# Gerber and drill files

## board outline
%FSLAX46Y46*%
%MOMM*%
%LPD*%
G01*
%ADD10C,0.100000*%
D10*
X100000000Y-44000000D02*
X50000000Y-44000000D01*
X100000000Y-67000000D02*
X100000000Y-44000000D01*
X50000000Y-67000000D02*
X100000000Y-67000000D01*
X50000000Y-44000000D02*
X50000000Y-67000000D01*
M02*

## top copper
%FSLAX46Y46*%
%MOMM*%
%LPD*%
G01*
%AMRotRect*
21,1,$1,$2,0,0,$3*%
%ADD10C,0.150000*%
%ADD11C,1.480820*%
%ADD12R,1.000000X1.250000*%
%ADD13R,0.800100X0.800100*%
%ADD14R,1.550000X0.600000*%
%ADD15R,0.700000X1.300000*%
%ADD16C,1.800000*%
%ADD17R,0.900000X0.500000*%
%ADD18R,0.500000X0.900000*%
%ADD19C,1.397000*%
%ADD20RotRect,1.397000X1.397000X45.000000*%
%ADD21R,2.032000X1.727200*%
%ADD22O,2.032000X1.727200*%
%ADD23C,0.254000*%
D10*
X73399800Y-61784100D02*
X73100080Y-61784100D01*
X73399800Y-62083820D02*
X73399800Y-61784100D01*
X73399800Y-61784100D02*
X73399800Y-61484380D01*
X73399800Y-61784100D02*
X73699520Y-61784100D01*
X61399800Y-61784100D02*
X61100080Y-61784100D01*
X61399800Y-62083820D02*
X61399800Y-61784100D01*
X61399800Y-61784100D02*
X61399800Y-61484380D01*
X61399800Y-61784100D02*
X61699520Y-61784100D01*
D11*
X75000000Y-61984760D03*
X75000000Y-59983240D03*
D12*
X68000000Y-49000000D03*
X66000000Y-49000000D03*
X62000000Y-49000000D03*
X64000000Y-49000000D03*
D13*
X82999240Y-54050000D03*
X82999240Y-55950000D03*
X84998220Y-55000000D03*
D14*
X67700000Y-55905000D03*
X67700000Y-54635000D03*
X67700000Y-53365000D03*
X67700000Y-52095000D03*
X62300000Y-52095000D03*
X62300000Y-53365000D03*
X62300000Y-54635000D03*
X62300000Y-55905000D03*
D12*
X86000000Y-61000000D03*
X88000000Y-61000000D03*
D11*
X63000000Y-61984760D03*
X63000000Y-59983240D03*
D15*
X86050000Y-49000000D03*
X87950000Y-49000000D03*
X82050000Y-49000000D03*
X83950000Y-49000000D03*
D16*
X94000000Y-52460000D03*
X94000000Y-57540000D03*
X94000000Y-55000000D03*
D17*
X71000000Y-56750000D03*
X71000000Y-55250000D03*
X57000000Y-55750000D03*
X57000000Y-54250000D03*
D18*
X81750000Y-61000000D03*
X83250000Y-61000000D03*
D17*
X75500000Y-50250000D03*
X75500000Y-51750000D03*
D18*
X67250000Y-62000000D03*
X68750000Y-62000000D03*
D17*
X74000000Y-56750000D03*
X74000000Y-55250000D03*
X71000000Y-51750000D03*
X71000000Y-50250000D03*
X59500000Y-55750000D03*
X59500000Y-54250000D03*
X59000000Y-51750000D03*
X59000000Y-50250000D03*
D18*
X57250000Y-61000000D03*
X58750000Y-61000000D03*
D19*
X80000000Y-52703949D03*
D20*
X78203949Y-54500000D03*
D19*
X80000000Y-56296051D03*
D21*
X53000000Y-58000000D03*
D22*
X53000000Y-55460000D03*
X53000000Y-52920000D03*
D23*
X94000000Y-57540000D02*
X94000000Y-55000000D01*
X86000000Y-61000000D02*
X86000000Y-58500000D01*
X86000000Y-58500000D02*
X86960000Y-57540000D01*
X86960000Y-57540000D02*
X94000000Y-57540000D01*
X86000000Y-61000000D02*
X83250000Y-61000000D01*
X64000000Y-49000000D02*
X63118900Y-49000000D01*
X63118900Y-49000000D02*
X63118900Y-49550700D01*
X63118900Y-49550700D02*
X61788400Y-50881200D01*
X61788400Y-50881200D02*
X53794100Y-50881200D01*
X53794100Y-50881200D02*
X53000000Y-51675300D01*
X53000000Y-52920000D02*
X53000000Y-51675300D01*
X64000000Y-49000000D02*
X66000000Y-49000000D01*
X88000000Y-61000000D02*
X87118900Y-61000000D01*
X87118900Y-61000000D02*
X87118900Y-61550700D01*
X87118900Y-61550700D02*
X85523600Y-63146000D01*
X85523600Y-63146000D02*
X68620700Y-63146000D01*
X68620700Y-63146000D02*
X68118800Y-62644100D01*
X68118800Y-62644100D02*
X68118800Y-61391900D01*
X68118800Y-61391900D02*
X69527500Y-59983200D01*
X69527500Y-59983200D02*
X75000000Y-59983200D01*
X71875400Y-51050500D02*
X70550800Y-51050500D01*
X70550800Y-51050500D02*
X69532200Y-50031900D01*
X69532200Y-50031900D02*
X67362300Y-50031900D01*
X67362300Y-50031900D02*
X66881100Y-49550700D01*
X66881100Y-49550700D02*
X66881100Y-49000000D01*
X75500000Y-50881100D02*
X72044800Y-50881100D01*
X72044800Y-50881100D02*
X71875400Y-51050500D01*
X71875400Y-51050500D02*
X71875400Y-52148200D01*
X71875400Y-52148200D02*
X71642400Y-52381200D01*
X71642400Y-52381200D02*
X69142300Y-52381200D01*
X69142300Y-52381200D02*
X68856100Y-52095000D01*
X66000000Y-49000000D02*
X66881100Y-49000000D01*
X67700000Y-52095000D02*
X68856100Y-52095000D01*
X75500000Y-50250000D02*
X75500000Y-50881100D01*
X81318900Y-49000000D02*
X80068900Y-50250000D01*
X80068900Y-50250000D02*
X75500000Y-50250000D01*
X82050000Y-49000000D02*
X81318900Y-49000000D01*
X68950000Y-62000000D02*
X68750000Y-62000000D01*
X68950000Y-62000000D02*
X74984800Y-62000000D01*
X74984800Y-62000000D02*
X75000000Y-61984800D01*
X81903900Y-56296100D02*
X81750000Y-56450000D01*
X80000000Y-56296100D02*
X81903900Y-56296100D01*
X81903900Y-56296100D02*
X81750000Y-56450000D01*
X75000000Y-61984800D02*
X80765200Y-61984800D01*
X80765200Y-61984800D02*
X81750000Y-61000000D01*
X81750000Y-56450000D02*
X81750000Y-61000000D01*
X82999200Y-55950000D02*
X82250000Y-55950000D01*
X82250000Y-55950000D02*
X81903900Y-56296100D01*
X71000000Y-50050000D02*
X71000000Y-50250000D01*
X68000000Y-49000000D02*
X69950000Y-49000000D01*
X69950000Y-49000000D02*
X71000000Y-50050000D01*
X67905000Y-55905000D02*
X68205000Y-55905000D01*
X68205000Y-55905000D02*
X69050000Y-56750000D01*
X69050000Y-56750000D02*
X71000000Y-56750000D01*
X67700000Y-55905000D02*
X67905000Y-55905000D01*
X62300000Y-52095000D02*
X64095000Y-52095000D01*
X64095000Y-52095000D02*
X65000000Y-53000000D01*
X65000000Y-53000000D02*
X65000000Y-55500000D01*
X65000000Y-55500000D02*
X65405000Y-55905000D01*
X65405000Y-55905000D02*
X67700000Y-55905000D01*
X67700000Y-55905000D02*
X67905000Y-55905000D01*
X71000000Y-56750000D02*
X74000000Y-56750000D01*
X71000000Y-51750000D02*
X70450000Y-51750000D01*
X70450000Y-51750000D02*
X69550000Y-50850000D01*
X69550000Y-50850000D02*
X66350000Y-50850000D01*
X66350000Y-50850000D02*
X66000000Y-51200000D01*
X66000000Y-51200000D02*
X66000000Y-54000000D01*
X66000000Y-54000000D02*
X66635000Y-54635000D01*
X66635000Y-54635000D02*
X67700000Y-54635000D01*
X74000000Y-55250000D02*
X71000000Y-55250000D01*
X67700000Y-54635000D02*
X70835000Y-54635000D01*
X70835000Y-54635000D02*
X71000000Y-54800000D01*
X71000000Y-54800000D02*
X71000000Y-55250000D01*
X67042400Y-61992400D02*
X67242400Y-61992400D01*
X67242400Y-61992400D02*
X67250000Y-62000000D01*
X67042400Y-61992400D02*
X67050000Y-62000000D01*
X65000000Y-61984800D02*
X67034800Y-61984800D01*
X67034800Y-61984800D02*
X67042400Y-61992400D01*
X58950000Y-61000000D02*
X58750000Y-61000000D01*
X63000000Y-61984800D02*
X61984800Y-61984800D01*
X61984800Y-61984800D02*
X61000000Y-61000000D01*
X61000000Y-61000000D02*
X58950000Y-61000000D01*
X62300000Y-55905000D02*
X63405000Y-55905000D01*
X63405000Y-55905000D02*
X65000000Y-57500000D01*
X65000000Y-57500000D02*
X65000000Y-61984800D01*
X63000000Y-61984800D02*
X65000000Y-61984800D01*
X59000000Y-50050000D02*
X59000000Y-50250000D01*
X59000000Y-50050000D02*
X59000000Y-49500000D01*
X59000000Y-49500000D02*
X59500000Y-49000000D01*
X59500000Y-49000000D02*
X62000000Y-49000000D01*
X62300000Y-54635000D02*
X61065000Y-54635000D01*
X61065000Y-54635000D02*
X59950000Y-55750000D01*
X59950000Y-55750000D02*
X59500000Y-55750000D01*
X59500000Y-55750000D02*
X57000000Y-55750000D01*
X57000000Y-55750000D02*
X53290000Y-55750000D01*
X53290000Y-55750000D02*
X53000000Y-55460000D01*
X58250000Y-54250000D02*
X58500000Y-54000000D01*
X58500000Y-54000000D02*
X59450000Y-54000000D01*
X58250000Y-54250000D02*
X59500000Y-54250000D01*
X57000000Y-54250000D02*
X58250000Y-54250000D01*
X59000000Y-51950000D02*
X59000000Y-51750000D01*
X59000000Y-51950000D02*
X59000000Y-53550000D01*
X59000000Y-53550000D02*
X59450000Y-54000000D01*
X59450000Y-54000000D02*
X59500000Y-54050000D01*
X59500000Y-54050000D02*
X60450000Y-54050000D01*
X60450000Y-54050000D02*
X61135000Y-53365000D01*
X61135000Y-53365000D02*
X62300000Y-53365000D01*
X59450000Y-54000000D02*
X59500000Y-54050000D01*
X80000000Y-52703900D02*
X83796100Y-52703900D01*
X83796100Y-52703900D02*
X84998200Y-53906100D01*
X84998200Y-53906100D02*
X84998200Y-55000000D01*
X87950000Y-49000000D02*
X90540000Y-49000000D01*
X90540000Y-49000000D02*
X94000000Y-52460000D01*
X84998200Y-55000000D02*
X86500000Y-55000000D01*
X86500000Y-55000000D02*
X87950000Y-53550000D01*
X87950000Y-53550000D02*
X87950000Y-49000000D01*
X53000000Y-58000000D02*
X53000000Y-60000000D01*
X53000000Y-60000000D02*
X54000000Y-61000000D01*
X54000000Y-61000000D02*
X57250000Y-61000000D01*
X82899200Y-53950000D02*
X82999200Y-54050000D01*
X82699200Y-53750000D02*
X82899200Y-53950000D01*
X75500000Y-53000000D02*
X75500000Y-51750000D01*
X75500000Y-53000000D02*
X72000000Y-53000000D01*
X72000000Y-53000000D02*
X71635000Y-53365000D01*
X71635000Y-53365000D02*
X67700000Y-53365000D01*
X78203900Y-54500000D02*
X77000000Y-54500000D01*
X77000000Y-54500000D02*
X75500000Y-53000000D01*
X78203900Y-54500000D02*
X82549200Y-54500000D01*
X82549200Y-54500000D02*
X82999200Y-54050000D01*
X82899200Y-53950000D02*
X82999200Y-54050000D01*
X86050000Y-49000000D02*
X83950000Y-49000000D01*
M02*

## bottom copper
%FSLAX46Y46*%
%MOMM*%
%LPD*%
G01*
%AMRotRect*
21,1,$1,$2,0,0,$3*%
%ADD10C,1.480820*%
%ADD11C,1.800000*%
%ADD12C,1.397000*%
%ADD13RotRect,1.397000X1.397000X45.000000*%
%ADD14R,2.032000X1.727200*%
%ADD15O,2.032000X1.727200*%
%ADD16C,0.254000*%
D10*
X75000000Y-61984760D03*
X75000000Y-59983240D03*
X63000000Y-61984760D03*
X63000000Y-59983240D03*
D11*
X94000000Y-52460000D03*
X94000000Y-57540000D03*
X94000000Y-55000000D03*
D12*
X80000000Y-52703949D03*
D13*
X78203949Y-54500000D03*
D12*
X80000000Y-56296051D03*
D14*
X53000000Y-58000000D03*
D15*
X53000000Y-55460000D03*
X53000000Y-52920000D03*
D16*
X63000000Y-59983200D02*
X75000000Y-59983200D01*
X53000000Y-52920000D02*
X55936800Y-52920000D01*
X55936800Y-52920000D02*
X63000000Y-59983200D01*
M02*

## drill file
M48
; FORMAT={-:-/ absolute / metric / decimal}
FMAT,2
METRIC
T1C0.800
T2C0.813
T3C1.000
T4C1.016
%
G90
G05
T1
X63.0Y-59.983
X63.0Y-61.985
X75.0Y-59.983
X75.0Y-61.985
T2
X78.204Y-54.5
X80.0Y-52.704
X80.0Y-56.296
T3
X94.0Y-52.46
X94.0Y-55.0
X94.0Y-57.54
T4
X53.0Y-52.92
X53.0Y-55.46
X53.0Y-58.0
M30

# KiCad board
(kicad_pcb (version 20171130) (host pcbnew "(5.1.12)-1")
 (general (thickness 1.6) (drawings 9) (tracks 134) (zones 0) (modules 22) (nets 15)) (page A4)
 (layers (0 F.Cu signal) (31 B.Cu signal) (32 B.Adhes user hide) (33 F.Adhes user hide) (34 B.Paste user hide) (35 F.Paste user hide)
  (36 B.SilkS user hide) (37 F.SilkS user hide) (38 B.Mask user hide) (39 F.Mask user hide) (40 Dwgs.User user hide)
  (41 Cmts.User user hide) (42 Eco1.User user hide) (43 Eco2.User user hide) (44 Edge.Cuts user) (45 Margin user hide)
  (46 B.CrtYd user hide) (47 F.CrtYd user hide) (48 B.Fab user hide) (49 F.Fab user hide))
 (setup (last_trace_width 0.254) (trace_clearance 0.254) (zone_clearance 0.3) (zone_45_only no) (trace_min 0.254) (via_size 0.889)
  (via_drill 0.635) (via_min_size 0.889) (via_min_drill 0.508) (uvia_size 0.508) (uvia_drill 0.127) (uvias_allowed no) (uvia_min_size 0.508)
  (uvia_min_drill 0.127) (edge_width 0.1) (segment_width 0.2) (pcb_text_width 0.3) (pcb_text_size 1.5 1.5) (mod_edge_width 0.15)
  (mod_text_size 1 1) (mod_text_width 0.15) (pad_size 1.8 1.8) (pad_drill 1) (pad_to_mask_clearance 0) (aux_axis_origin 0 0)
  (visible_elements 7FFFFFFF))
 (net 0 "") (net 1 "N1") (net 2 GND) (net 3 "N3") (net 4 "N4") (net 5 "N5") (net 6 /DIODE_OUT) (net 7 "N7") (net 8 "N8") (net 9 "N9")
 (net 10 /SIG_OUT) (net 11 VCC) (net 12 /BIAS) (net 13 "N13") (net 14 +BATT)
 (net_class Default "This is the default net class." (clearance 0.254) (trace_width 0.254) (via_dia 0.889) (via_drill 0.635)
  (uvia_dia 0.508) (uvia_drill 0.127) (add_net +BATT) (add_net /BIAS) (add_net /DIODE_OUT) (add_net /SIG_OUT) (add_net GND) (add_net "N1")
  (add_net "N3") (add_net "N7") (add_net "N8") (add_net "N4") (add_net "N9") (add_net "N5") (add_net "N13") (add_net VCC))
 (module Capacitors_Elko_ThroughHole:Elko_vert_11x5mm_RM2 (layer F.Cu) (at 75 62 90)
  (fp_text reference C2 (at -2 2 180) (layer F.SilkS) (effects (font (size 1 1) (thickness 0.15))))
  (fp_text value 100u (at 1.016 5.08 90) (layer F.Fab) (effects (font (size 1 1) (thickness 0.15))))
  (fp_line (start 0.2159 -1.6002) (end 0.2159 -1.89992) (layer F.Cu) (width 0.15))
  (fp_line (start -0.08382 -1.6002) (end 0.2159 -1.6002) (layer F.Cu) (width 0.15))
  (fp_line (start 0.2159 -1.6002) (end 0.51562 -1.6002) (layer F.Cu) (width 0.15))
  (fp_line (start 0.2159 -1.6002) (end 0.2159 -1.30048) (layer F.Cu) (width 0.15))
  (pad 1 thru_hole circle (at 0.01524 0 90) (size 1.48082 1.48082) (drill 0.8001) (layers *.Cu *.Mask F.SilkS) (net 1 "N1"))
  (pad 2 thru_hole circle (at 2.01676 0 90) (size 1.48082 1.48082) (drill 0.8001) (layers *.Cu *.Mask F.SilkS) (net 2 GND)))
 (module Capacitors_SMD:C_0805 (layer F.Cu) (at 67 49 180)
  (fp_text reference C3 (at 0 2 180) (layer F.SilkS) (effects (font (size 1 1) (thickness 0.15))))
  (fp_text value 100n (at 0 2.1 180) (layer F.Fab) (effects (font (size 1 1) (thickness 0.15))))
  (pad 1 smd rect (at -1 0 180) (size 1 1.25) (layers F.Cu F.Paste F.Mask) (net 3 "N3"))
  (pad 2 smd rect (at 1 0 180) (size 1 1.25) (layers F.Cu F.Paste F.Mask) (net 2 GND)))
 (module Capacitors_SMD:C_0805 (layer F.Cu) (at 63 49)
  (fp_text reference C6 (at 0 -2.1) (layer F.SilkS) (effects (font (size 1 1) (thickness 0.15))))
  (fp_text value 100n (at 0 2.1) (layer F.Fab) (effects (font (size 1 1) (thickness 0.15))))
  (pad 1 smd rect (at -1 0) (size 1 1.25) (layers F.Cu F.Paste F.Mask) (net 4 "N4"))
  (pad 2 smd rect (at 1 0) (size 1 1.25) (layers F.Cu F.Paste F.Mask) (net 2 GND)))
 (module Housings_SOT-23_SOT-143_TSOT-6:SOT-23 (layer F.Cu) (at 84 55 270)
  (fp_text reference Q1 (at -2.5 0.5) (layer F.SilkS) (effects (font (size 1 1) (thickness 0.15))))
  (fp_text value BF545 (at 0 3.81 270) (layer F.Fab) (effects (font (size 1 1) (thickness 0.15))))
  (pad 1 smd rect (at -0.95 1.00076 270) (size 0.8001 0.8001) (layers F.Cu F.Paste F.Mask) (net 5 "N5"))
  (pad 2 smd rect (at 0.95 1.00076 270) (size 0.8001 0.8001) (layers F.Cu F.Paste F.Mask) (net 1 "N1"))
  (pad 3 smd rect (at 0 -0.99822 270) (size 0.8001 0.8001) (layers F.Cu F.Paste F.Mask) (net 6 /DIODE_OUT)))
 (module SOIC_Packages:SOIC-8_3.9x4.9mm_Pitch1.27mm (layer F.Cu) (at 65 54 180)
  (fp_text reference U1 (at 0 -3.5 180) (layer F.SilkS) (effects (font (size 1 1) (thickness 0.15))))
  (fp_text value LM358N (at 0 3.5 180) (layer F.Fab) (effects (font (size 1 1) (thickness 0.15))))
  (pad 1 smd rect (at -2.7 -1.905 180) (size 1.55 0.6) (layers F.Cu F.Paste F.Mask) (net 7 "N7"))
  (pad 2 smd rect (at -2.7 -0.635 180) (size 1.55 0.6) (layers F.Cu F.Paste F.Mask) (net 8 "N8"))
  (pad 3 smd rect (at -2.7 0.635 180) (size 1.55 0.6) (layers F.Cu F.Paste F.Mask) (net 5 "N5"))
  (pad 4 smd rect (at -2.7 1.905 180) (size 1.55 0.6) (layers F.Cu F.Paste F.Mask) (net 2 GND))
  (pad 5 smd rect (at 2.7 1.905 180) (size 1.55 0.6) (layers F.Cu F.Paste F.Mask) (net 7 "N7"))
  (pad 6 smd rect (at 2.7 0.635 180) (size 1.55 0.6) (layers F.Cu F.Paste F.Mask) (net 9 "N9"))
  (pad 7 smd rect (at 2.7 -0.635 180) (size 1.55 0.6) (layers F.Cu F.Paste F.Mask) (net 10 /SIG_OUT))
  (pad 8 smd rect (at 2.7 -1.905 180) (size 1.55 0.6) (layers F.Cu F.Paste F.Mask) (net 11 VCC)))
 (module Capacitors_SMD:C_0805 (layer F.Cu) (at 87 61)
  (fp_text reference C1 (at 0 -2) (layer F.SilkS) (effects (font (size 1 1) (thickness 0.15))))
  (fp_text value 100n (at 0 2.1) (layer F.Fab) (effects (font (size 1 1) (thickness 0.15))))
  (pad 1 smd rect (at -1 0) (size 1 1.25) (layers F.Cu F.Paste F.Mask) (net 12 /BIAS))
  (pad 2 smd rect (at 1 0) (size 1 1.25) (layers F.Cu F.Paste F.Mask) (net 2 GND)))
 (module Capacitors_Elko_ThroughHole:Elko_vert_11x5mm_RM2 (layer F.Cu) (at 63 62 90)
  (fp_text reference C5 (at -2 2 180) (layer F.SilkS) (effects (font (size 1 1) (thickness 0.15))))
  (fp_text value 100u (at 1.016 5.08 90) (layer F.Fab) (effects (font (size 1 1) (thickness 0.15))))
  (fp_line (start 0.2159 -1.6002) (end 0.2159 -1.89992) (layer F.Cu) (width 0.15))
  (fp_line (start -0.08382 -1.6002) (end 0.2159 -1.6002) (layer F.Cu) (width 0.15))
  (fp_line (start 0.2159 -1.6002) (end 0.51562 -1.6002) (layer F.Cu) (width 0.15))
  (fp_line (start 0.2159 -1.6002) (end 0.2159 -1.30048) (layer F.Cu) (width 0.15))
  (pad 1 thru_hole circle (at 0.01524 0 90) (size 1.48082 1.48082) (drill 0.8001) (layers *.Cu *.Mask F.SilkS) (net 11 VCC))
  (pad 2 thru_hole circle (at 2.01676 0 90) (size 1.48082 1.48082) (drill 0.8001) (layers *.Cu *.Mask F.SilkS) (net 2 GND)))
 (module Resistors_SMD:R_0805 (layer F.Cu) (at 87 49)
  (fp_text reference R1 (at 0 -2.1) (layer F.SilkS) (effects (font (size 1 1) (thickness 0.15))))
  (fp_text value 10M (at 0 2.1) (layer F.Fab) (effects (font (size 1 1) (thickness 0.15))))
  (pad 1 smd rect (at -0.95 0) (size 0.7 1.3) (layers F.Cu F.Paste F.Mask) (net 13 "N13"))
  (pad 2 smd rect (at 0.95 0) (size 0.7 1.3) (layers F.Cu F.Paste F.Mask) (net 6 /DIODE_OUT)))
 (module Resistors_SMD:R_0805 (layer F.Cu) (at 83 49)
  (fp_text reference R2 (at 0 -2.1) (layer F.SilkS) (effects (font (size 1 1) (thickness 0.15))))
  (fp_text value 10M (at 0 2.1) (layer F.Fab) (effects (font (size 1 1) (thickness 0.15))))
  (pad 1 smd rect (at -0.95 0) (size 0.7 1.3) (layers F.Cu F.Paste F.Mask) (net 2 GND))
  (pad 2 smd rect (at 0.95 0) (size 0.7 1.3) (layers F.Cu F.Paste F.Mask) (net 13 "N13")))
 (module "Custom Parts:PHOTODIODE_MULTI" (layer F.Cu) (at 94 55)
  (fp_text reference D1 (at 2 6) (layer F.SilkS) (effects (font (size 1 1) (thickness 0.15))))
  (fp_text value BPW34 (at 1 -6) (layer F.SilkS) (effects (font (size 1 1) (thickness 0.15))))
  (pad 1 thru_hole circle (at 0 -2.54) (size 1.8 1.8) (drill 1) (layers *.Cu *.Mask F.SilkS) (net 6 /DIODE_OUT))
  (pad 2 thru_hole circle (at 0 2.54) (size 1.8 1.8) (drill 1) (layers *.Cu *.Mask F.SilkS) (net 12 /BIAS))
  (pad 2 thru_hole circle (at 0 0) (size 1.8 1.8) (drill 1) (layers *.Cu *.Mask F.SilkS) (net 12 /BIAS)))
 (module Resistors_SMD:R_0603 (layer F.Cu) (at 71 56 90)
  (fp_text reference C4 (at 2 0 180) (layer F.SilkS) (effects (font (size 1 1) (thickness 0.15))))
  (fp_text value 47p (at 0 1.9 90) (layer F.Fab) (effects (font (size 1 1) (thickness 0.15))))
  (pad 1 smd rect (at -0.75 0 90) (size 0.5 0.9) (layers F.Cu F.Paste F.Mask) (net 7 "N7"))
  (pad 2 smd rect (at 0.75 0 90) (size 0.5 0.9) (layers F.Cu F.Paste F.Mask) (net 8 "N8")))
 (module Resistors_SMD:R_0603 (layer F.Cu) (at 57 55 90)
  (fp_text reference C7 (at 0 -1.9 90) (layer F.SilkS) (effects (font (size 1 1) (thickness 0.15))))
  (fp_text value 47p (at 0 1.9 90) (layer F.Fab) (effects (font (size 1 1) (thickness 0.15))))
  (pad 1 smd rect (at -0.75 0 90) (size 0.5 0.9) (layers F.Cu F.Paste F.Mask) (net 10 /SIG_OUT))
  (pad 2 smd rect (at 0.75 0 90) (size 0.5 0.9) (layers F.Cu F.Paste F.Mask) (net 9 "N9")))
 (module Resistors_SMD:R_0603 (layer F.Cu) (at 82.5 61)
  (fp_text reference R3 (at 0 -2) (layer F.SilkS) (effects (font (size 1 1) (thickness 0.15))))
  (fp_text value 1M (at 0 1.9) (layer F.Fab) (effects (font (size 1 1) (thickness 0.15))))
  (pad 1 smd rect (at -0.75 0) (size 0.5 0.9) (layers F.Cu F.Paste F.Mask) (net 1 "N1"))
  (pad 2 smd rect (at 0.75 0) (size 0.5 0.9) (layers F.Cu F.Paste F.Mask) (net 12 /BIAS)))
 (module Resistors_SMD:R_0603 (layer F.Cu) (at 75.5 51 270)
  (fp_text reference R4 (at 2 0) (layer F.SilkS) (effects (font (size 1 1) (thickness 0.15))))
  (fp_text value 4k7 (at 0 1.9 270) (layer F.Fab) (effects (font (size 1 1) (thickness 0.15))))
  (pad 1 smd rect (at -0.75 0 270) (size 0.5 0.9) (layers F.Cu F.Paste F.Mask) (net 2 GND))
  (pad 2 smd rect (at 0.75 0 270) (size 0.5 0.9) (layers F.Cu F.Paste F.Mask) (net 5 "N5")))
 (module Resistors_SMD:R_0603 (layer F.Cu) (at 68 62)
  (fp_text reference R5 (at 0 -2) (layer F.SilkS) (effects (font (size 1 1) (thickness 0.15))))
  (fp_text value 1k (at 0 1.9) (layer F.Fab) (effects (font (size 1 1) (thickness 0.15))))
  (pad 1 smd rect (at -0.75 0) (size 0.5 0.9) (layers F.Cu F.Paste F.Mask) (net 11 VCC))
  (pad 2 smd rect (at 0.75 0) (size 0.5 0.9) (layers F.Cu F.Paste F.Mask) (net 1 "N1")))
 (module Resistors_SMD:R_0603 (layer F.Cu) (at 74 56 90)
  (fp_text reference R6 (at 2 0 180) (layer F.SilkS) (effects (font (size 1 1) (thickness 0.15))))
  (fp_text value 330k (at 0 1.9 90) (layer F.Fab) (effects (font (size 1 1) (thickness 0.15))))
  (pad 1 smd rect (at -0.75 0 90) (size 0.5 0.9) (layers F.Cu F.Paste F.Mask) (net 7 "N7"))
  (pad 2 smd rect (at 0.75 0 90) (size 0.5 0.9) (layers F.Cu F.Paste F.Mask) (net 8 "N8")))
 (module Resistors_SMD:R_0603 (layer F.Cu) (at 71 51 90)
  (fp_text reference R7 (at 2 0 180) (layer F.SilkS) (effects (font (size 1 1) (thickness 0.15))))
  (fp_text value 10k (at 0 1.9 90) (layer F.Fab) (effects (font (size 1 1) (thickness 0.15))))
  (pad 1 smd rect (at -0.75 0 90) (size 0.5 0.9) (layers F.Cu F.Paste F.Mask) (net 8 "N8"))
  (pad 2 smd rect (at 0.75 0 90) (size 0.5 0.9) (layers F.Cu F.Paste F.Mask) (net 3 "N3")))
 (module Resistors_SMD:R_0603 (layer F.Cu) (at 59.5 55 90)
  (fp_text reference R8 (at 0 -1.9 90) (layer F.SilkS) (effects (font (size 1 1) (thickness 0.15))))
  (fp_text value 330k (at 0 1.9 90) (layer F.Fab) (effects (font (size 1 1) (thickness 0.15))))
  (pad 1 smd rect (at -0.75 0 90) (size 0.5 0.9) (layers F.Cu F.Paste F.Mask) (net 10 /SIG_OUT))
  (pad 2 smd rect (at 0.75 0 90) (size 0.5 0.9) (layers F.Cu F.Paste F.Mask) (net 9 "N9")))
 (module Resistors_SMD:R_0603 (layer F.Cu) (at 59 51 90)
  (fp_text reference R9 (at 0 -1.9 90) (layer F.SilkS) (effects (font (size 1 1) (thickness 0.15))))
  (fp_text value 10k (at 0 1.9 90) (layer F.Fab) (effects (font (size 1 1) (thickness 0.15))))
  (pad 1 smd rect (at -0.75 0 90) (size 0.5 0.9) (layers F.Cu F.Paste F.Mask) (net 9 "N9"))
  (pad 2 smd rect (at 0.75 0 90) (size 0.5 0.9) (layers F.Cu F.Paste F.Mask) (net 4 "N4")))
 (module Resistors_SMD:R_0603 (layer F.Cu) (at 58 61)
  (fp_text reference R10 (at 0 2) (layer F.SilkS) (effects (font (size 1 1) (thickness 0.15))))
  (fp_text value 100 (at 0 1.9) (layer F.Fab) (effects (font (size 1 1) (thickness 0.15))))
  (pad 1 smd rect (at -0.75 0) (size 0.5 0.9) (layers F.Cu F.Paste F.Mask) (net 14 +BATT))
  (pad 2 smd rect (at 0.75 0) (size 0.5 0.9) (layers F.Cu F.Paste F.Mask) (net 11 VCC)))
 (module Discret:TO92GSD (layer F.Cu) (at 80 54.5 45)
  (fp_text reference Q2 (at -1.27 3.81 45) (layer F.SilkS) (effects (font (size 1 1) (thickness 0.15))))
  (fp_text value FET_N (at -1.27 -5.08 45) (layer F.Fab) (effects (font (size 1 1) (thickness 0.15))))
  (pad G thru_hole circle (at 1.27 -1.27 45) (size 1.397 1.397) (drill 0.8128) (layers *.Cu *.Mask F.SilkS) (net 6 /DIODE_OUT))
  (pad S thru_hole rect (at -1.27 -1.27 45) (size 1.397 1.397) (drill 0.8128) (layers *.Cu *.Mask F.SilkS) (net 5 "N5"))
  (pad D thru_hole circle (at -1.27 1.27 45) (size 1.397 1.397) (drill 0.8128) (layers *.Cu *.Mask F.SilkS) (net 1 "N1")))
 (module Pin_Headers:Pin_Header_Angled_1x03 (layer F.Cu) (at 53 58 180)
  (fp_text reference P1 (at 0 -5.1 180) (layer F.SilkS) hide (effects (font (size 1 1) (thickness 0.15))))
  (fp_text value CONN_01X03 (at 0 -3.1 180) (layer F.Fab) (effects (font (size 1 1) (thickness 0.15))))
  (pad 1 thru_hole rect (at 0 0 180) (size 2.032 1.7272) (drill 1.016) (layers *.Cu *.Mask F.SilkS) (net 14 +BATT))
  (pad 2 thru_hole oval (at 0 2.54 180) (size 2.032 1.7272) (drill 1.016) (layers *.Cu *.Mask F.SilkS) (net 10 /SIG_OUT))
  (pad 3 thru_hole oval (at 0 5.08 180) (size 2.032 1.7272) (drill 1.016) (layers *.Cu *.Mask F.SilkS) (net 2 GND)))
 (gr_line (start 100 44) (end 50 44) (angle 90) (layer Edge.Cuts) (width 0.1))
 (gr_line (start 100 67) (end 100 44) (angle 90) (layer Edge.Cuts) (width 0.1))
 (gr_line (start 50 67) (end 100 67) (angle 90) (layer Edge.Cuts) (width 0.1))
 (gr_line (start 50 44) (end 50 67) (angle 90) (layer Edge.Cuts) (width 0.1))
 (segment (start 94 57.54) (end 94 55) (width 0.254) (layer F.Cu) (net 12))
 (segment (start 86 61) (end 86 58.5) (width 0.254) (layer F.Cu) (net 12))
 (segment (start 86 58.5) (end 86.96 57.54) (width 0.254) (layer F.Cu) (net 12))
 (segment (start 86.96 57.54) (end 94 57.54) (width 0.254) (layer F.Cu) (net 12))
 (segment (start 86 61) (end 83.25 61) (width 0.254) (layer F.Cu) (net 12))
 (segment (start 63 59.9832) (end 75 59.9832) (width 0.254) (layer B.Cu) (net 2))
 (segment (start 53 52.92) (end 55.9368 52.92) (width 0.254) (layer B.Cu) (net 2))
 (segment (start 55.9368 52.92) (end 63 59.9832) (width 0.254) (layer B.Cu) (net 2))
 (segment (start 64 49) (end 63.1189 49) (width 0.254) (layer F.Cu) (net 2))
 (segment (start 63.1189 49) (end 63.1189 49.5507) (width 0.254) (layer F.Cu) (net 2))
 (segment (start 63.1189 49.5507) (end 61.7884 50.8812) (width 0.254) (layer F.Cu) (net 2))
 (segment (start 61.7884 50.8812) (end 53.7941 50.8812) (width 0.254) (layer F.Cu) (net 2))
 (segment (start 53.7941 50.8812) (end 53 51.6753) (width 0.254) (layer F.Cu) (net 2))
 (segment (start 53 52.92) (end 53 51.6753) (width 0.254) (layer F.Cu) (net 2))
 (segment (start 64 49) (end 66 49) (width 0.254) (layer F.Cu) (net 2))
 (segment (start 88 61) (end 87.1189 61) (width 0.254) (layer F.Cu) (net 2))
 (segment (start 87.1189 61) (end 87.1189 61.5507) (width 0.254) (layer F.Cu) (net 2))
 (segment (start 87.1189 61.5507) (end 85.5236 63.146) (width 0.254) (layer F.Cu) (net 2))
 (segment (start 85.5236 63.146) (end 68.6207 63.146) (width 0.254) (layer F.Cu) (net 2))
 (segment (start 68.6207 63.146) (end 68.1188 62.6441) (width 0.254) (layer F.Cu) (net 2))
 (segment (start 68.1188 62.6441) (end 68.1188 61.3919) (width 0.254) (layer F.Cu) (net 2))
 (segment (start 68.1188 61.3919) (end 69.5275 59.9832) (width 0.254) (layer F.Cu) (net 2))
 (segment (start 69.5275 59.9832) (end 75 59.9832) (width 0.254) (layer F.Cu) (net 2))
 (segment (start 71.8754 51.0505) (end 70.5508 51.0505) (width 0.254) (layer F.Cu) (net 2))
 (segment (start 70.5508 51.0505) (end 69.5322 50.0319) (width 0.254) (layer F.Cu) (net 2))
 (segment (start 69.5322 50.0319) (end 67.3623 50.0319) (width 0.254) (layer F.Cu) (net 2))
 (segment (start 67.3623 50.0319) (end 66.8811 49.5507) (width 0.254) (layer F.Cu) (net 2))
 (segment (start 66.8811 49.5507) (end 66.8811 49) (width 0.254) (layer F.Cu) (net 2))
 (segment (start 75.5 50.8811) (end 72.0448 50.8811) (width 0.254) (layer F.Cu) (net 2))
 (segment (start 72.0448 50.8811) (end 71.8754 51.0505) (width 0.254) (layer F.Cu) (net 2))
 (segment (start 71.8754 51.0505) (end 71.8754 52.1482) (width 0.254) (layer F.Cu) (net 2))
 (segment (start 71.8754 52.1482) (end 71.6424 52.3812) (width 0.254) (layer F.Cu) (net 2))
 (segment (start 71.6424 52.3812) (end 69.1423 52.3812) (width 0.254) (layer F.Cu) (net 2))
 (segment (start 69.1423 52.3812) (end 68.8561 52.095) (width 0.254) (layer F.Cu) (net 2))
 (segment (start 66 49) (end 66.8811 49) (width 0.254) (layer F.Cu) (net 2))
 (segment (start 67.7 52.095) (end 68.8561 52.095) (width 0.254) (layer F.Cu) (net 2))
 (segment (start 75.5 50.25) (end 75.5 50.8811) (width 0.254) (layer F.Cu) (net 2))
 (segment (start 81.3189 49) (end 80.0689 50.25) (width 0.254) (layer F.Cu) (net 2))
 (segment (start 80.0689 50.25) (end 75.5 50.25) (width 0.254) (layer F.Cu) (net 2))
 (segment (start 82.05 49) (end 81.3189 49) (width 0.254) (layer F.Cu) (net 2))
 (segment (start 68.95 62) (end 68.75 62) (width 0.254) (layer F.Cu) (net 1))
 (segment (start 68.95 62) (end 74.9848 62) (width 0.254) (layer F.Cu) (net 1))
 (segment (start 74.9848 62) (end 75 61.9848) (width 0.254) (layer F.Cu) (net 1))
 (segment (start 81.9039 56.2961) (end 81.75 56.45) (width 0.254) (layer F.Cu) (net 1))
 (segment (start 80 56.2961) (end 81.9039 56.2961) (width 0.254) (layer F.Cu) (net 1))
 (segment (start 81.9039 56.2961) (end 81.75 56.45) (width 0.254) (layer F.Cu) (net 1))
 (segment (start 75 61.9848) (end 80.7652 61.9848) (width 0.254) (layer F.Cu) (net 1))
 (segment (start 80.7652 61.9848) (end 81.75 61) (width 0.254) (layer F.Cu) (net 1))
 (segment (start 81.75 56.45) (end 81.75 61) (width 0.254) (layer F.Cu) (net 1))
 (segment (start 82.9992 55.95) (end 82.25 55.95) (width 0.254) (layer F.Cu) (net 1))
 (segment (start 82.25 55.95) (end 81.9039 56.2961) (width 0.254) (layer F.Cu) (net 1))
 (segment (start 71 50.05) (end 71 50.25) (width 0.254) (layer F.Cu) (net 3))
 (segment (start 68 49) (end 69.95 49) (width 0.254) (layer F.Cu) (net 3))
 (segment (start 69.95 49) (end 71 50.05) (width 0.254) (layer F.Cu) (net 3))
 (segment (start 67.905 55.905) (end 68.205 55.905) (width 0.254) (layer F.Cu) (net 7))
 (segment (start 68.205 55.905) (end 69.05 56.75) (width 0.254) (layer F.Cu) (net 7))
 (segment (start 69.05 56.75) (end 71 56.75) (width 0.254) (layer F.Cu) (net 7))
 (segment (start 67.7 55.905) (end 67.905 55.905) (width 0.254) (layer F.Cu) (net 7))
 (segment (start 62.3 52.095) (end 64.095 52.095) (width 0.254) (layer F.Cu) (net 7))
 (segment (start 64.095 52.095) (end 65 53) (width 0.254) (layer F.Cu) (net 7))
 (segment (start 65 53) (end 65 55.5) (width 0.254) (layer F.Cu) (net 7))
 (segment (start 65 55.5) (end 65.405 55.905) (width 0.254) (layer F.Cu) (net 7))
 (segment (start 65.405 55.905) (end 67.7 55.905) (width 0.254) (layer F.Cu) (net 7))
 (segment (start 67.7 55.905) (end 67.905 55.905) (width 0.254) (layer F.Cu) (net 7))
 (segment (start 71 56.75) (end 74 56.75) (width 0.254) (layer F.Cu) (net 7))
 (segment (start 71 51.75) (end 70.45 51.75) (width 0.254) (layer F.Cu) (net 8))
 (segment (start 70.45 51.75) (end 69.55 50.85) (width 0.254) (layer F.Cu) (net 8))
 (segment (start 69.55 50.85) (end 66.35 50.85) (width 0.254) (layer F.Cu) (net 8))
 (segment (start 66.35 50.85) (end 66 51.2) (width 0.254) (layer F.Cu) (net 8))
 (segment (start 66 51.2) (end 66 54) (width 0.254) (layer F.Cu) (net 8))
 (segment (start 66 54) (end 66.635 54.635) (width 0.254) (layer F.Cu) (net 8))
 (segment (start 66.635 54.635) (end 67.7 54.635) (width 0.254) (layer F.Cu) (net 8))
 (segment (start 74 55.25) (end 71 55.25) (width 0.254) (layer F.Cu) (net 8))
 (segment (start 67.7 54.635) (end 70.835 54.635) (width 0.254) (layer F.Cu) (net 8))
 (segment (start 70.835 54.635) (end 71 54.8) (width 0.254) (layer F.Cu) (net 8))
 (segment (start 71 54.8) (end 71 55.25) (width 0.254) (layer F.Cu) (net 8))
 (segment (start 67.0424 61.9924) (end 67.2424 61.9924) (width 0.254) (layer F.Cu) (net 11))
 (segment (start 67.2424 61.9924) (end 67.25 62) (width 0.254) (layer F.Cu) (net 11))
 (segment (start 67.0424 61.9924) (end 67.05 62) (width 0.254) (layer F.Cu) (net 11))
 (segment (start 65 61.9848) (end 67.0348 61.9848) (width 0.254) (layer F.Cu) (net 11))
 (segment (start 67.0348 61.9848) (end 67.0424 61.9924) (width 0.254) (layer F.Cu) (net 11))
 (segment (start 58.95 61) (end 58.75 61) (width 0.254) (layer F.Cu) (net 11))
 (segment (start 63 61.9848) (end 61.9848 61.9848) (width 0.254) (layer F.Cu) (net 11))
 (segment (start 61.9848 61.9848) (end 61 61) (width 0.254) (layer F.Cu) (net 11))
 (segment (start 61 61) (end 58.95 61) (width 0.254) (layer F.Cu) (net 11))
 (segment (start 62.3 55.905) (end 63.405 55.905) (width 0.254) (layer F.Cu) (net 11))
 (segment (start 63.405 55.905) (end 65 57.5) (width 0.254) (layer F.Cu) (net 11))
 (segment (start 65 57.5) (end 65 61.9848) (width 0.254) (layer F.Cu) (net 11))
 (segment (start 63 61.9848) (end 65 61.9848) (width 0.254) (layer F.Cu) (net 11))
 (segment (start 59 50.05) (end 59 50.25) (width 0.254) (layer F.Cu) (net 4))
 (segment (start 59 50.05) (end 59 49.5) (width 0.254) (layer F.Cu) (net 4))
 (segment (start 59 49.5) (end 59.5 49) (width 0.254) (layer F.Cu) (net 4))
 (segment (start 59.5 49) (end 62 49) (width 0.254) (layer F.Cu) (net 4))
 (segment (start 62.3 54.635) (end 61.065 54.635) (width 0.254) (layer F.Cu) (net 10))
 (segment (start 61.065 54.635) (end 59.95 55.75) (width 0.254) (layer F.Cu) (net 10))
 (segment (start 59.95 55.75) (end 59.5 55.75) (width 0.254) (layer F.Cu) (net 10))
 (segment (start 59.5 55.75) (end 57 55.75) (width 0.254) (layer F.Cu) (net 10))
 (segment (start 57 55.75) (end 53.29 55.75) (width 0.254) (layer F.Cu) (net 10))
 (segment (start 53.29 55.75) (end 53 55.46) (width 0.254) (layer F.Cu) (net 10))
 (segment (start 58.25 54.25) (end 58.5 54) (width 0.254) (layer F.Cu) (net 9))
 (segment (start 58.5 54) (end 59.45 54) (width 0.254) (layer F.Cu) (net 9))
 (segment (start 58.25 54.25) (end 59.5 54.25) (width 0.254) (layer F.Cu) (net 9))
 (segment (start 57 54.25) (end 58.25 54.25) (width 0.254) (layer F.Cu) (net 9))
 (segment (start 59 51.95) (end 59 51.75) (width 0.254) (layer F.Cu) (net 9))
 (segment (start 59 51.95) (end 59 53.55) (width 0.254) (layer F.Cu) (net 9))
 (segment (start 59 53.55) (end 59.45 54) (width 0.254) (layer F.Cu) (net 9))
 (segment (start 59.45 54) (end 59.5 54.05) (width 0.254) (layer F.Cu) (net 9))
 (segment (start 59.5 54.05) (end 60.45 54.05) (width 0.254) (layer F.Cu) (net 9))
 (segment (start 60.45 54.05) (end 61.135 53.365) (width 0.254) (layer F.Cu) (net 9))
 (segment (start 61.135 53.365) (end 62.3 53.365) (width 0.254) (layer F.Cu) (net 9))
 (segment (start 59.45 54) (end 59.5 54.05) (width 0.254) (layer F.Cu) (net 9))
 (segment (start 80 52.7039) (end 83.7961 52.7039) (width 0.254) (layer F.Cu) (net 6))
 (segment (start 83.7961 52.7039) (end 84.9982 53.9061) (width 0.254) (layer F.Cu) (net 6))
 (segment (start 84.9982 53.9061) (end 84.9982 55) (width 0.254) (layer F.Cu) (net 6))
 (segment (start 87.95 49) (end 90.54 49) (width 0.254) (layer F.Cu) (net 6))
 (segment (start 90.54 49) (end 94 52.46) (width 0.254) (layer F.Cu) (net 6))
 (segment (start 84.9982 55) (end 86.5 55) (width 0.254) (layer F.Cu) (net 6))
 (segment (start 86.5 55) (end 87.95 53.55) (width 0.254) (layer F.Cu) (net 6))
 (segment (start 87.95 53.55) (end 87.95 49) (width 0.254) (layer F.Cu) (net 6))
 (segment (start 53 58) (end 53 60) (width 0.254) (layer F.Cu) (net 14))
 (segment (start 53 60) (end 54 61) (width 0.254) (layer F.Cu) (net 14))
 (segment (start 54 61) (end 57.25 61) (width 0.254) (layer F.Cu) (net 14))
 (segment (start 82.8992 53.95) (end 82.9992 54.05) (width 0.254) (layer F.Cu) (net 5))
 (segment (start 82.6992 53.75) (end 82.8992 53.95) (width 0.254) (layer F.Cu) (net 5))
 (segment (start 75.5 53) (end 75.5 51.75) (width 0.254) (layer F.Cu) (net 5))
 (segment (start 75.5 53) (end 72 53) (width 0.254) (layer F.Cu) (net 5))
 (segment (start 72 53) (end 71.635 53.365) (width 0.254) (layer F.Cu) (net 5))
 (segment (start 71.635 53.365) (end 67.7 53.365) (width 0.254) (layer F.Cu) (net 5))
 (segment (start 78.2039 54.5) (end 77 54.5) (width 0.254) (layer F.Cu) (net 5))
 (segment (start 77 54.5) (end 75.5 53) (width 0.254) (layer F.Cu) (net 5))
 (segment (start 78.2039 54.5) (end 82.5492 54.5) (width 0.254) (layer F.Cu) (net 5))
 (segment (start 82.5492 54.5) (end 82.9992 54.05) (width 0.254) (layer F.Cu) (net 5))
 (segment (start 82.8992 53.95) (end 82.9992 54.05) (width 0.254) (layer F.Cu) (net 5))
 (segment (start 86.05 49) (end 83.95 49) (width 0.254) (layer F.Cu) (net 13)))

